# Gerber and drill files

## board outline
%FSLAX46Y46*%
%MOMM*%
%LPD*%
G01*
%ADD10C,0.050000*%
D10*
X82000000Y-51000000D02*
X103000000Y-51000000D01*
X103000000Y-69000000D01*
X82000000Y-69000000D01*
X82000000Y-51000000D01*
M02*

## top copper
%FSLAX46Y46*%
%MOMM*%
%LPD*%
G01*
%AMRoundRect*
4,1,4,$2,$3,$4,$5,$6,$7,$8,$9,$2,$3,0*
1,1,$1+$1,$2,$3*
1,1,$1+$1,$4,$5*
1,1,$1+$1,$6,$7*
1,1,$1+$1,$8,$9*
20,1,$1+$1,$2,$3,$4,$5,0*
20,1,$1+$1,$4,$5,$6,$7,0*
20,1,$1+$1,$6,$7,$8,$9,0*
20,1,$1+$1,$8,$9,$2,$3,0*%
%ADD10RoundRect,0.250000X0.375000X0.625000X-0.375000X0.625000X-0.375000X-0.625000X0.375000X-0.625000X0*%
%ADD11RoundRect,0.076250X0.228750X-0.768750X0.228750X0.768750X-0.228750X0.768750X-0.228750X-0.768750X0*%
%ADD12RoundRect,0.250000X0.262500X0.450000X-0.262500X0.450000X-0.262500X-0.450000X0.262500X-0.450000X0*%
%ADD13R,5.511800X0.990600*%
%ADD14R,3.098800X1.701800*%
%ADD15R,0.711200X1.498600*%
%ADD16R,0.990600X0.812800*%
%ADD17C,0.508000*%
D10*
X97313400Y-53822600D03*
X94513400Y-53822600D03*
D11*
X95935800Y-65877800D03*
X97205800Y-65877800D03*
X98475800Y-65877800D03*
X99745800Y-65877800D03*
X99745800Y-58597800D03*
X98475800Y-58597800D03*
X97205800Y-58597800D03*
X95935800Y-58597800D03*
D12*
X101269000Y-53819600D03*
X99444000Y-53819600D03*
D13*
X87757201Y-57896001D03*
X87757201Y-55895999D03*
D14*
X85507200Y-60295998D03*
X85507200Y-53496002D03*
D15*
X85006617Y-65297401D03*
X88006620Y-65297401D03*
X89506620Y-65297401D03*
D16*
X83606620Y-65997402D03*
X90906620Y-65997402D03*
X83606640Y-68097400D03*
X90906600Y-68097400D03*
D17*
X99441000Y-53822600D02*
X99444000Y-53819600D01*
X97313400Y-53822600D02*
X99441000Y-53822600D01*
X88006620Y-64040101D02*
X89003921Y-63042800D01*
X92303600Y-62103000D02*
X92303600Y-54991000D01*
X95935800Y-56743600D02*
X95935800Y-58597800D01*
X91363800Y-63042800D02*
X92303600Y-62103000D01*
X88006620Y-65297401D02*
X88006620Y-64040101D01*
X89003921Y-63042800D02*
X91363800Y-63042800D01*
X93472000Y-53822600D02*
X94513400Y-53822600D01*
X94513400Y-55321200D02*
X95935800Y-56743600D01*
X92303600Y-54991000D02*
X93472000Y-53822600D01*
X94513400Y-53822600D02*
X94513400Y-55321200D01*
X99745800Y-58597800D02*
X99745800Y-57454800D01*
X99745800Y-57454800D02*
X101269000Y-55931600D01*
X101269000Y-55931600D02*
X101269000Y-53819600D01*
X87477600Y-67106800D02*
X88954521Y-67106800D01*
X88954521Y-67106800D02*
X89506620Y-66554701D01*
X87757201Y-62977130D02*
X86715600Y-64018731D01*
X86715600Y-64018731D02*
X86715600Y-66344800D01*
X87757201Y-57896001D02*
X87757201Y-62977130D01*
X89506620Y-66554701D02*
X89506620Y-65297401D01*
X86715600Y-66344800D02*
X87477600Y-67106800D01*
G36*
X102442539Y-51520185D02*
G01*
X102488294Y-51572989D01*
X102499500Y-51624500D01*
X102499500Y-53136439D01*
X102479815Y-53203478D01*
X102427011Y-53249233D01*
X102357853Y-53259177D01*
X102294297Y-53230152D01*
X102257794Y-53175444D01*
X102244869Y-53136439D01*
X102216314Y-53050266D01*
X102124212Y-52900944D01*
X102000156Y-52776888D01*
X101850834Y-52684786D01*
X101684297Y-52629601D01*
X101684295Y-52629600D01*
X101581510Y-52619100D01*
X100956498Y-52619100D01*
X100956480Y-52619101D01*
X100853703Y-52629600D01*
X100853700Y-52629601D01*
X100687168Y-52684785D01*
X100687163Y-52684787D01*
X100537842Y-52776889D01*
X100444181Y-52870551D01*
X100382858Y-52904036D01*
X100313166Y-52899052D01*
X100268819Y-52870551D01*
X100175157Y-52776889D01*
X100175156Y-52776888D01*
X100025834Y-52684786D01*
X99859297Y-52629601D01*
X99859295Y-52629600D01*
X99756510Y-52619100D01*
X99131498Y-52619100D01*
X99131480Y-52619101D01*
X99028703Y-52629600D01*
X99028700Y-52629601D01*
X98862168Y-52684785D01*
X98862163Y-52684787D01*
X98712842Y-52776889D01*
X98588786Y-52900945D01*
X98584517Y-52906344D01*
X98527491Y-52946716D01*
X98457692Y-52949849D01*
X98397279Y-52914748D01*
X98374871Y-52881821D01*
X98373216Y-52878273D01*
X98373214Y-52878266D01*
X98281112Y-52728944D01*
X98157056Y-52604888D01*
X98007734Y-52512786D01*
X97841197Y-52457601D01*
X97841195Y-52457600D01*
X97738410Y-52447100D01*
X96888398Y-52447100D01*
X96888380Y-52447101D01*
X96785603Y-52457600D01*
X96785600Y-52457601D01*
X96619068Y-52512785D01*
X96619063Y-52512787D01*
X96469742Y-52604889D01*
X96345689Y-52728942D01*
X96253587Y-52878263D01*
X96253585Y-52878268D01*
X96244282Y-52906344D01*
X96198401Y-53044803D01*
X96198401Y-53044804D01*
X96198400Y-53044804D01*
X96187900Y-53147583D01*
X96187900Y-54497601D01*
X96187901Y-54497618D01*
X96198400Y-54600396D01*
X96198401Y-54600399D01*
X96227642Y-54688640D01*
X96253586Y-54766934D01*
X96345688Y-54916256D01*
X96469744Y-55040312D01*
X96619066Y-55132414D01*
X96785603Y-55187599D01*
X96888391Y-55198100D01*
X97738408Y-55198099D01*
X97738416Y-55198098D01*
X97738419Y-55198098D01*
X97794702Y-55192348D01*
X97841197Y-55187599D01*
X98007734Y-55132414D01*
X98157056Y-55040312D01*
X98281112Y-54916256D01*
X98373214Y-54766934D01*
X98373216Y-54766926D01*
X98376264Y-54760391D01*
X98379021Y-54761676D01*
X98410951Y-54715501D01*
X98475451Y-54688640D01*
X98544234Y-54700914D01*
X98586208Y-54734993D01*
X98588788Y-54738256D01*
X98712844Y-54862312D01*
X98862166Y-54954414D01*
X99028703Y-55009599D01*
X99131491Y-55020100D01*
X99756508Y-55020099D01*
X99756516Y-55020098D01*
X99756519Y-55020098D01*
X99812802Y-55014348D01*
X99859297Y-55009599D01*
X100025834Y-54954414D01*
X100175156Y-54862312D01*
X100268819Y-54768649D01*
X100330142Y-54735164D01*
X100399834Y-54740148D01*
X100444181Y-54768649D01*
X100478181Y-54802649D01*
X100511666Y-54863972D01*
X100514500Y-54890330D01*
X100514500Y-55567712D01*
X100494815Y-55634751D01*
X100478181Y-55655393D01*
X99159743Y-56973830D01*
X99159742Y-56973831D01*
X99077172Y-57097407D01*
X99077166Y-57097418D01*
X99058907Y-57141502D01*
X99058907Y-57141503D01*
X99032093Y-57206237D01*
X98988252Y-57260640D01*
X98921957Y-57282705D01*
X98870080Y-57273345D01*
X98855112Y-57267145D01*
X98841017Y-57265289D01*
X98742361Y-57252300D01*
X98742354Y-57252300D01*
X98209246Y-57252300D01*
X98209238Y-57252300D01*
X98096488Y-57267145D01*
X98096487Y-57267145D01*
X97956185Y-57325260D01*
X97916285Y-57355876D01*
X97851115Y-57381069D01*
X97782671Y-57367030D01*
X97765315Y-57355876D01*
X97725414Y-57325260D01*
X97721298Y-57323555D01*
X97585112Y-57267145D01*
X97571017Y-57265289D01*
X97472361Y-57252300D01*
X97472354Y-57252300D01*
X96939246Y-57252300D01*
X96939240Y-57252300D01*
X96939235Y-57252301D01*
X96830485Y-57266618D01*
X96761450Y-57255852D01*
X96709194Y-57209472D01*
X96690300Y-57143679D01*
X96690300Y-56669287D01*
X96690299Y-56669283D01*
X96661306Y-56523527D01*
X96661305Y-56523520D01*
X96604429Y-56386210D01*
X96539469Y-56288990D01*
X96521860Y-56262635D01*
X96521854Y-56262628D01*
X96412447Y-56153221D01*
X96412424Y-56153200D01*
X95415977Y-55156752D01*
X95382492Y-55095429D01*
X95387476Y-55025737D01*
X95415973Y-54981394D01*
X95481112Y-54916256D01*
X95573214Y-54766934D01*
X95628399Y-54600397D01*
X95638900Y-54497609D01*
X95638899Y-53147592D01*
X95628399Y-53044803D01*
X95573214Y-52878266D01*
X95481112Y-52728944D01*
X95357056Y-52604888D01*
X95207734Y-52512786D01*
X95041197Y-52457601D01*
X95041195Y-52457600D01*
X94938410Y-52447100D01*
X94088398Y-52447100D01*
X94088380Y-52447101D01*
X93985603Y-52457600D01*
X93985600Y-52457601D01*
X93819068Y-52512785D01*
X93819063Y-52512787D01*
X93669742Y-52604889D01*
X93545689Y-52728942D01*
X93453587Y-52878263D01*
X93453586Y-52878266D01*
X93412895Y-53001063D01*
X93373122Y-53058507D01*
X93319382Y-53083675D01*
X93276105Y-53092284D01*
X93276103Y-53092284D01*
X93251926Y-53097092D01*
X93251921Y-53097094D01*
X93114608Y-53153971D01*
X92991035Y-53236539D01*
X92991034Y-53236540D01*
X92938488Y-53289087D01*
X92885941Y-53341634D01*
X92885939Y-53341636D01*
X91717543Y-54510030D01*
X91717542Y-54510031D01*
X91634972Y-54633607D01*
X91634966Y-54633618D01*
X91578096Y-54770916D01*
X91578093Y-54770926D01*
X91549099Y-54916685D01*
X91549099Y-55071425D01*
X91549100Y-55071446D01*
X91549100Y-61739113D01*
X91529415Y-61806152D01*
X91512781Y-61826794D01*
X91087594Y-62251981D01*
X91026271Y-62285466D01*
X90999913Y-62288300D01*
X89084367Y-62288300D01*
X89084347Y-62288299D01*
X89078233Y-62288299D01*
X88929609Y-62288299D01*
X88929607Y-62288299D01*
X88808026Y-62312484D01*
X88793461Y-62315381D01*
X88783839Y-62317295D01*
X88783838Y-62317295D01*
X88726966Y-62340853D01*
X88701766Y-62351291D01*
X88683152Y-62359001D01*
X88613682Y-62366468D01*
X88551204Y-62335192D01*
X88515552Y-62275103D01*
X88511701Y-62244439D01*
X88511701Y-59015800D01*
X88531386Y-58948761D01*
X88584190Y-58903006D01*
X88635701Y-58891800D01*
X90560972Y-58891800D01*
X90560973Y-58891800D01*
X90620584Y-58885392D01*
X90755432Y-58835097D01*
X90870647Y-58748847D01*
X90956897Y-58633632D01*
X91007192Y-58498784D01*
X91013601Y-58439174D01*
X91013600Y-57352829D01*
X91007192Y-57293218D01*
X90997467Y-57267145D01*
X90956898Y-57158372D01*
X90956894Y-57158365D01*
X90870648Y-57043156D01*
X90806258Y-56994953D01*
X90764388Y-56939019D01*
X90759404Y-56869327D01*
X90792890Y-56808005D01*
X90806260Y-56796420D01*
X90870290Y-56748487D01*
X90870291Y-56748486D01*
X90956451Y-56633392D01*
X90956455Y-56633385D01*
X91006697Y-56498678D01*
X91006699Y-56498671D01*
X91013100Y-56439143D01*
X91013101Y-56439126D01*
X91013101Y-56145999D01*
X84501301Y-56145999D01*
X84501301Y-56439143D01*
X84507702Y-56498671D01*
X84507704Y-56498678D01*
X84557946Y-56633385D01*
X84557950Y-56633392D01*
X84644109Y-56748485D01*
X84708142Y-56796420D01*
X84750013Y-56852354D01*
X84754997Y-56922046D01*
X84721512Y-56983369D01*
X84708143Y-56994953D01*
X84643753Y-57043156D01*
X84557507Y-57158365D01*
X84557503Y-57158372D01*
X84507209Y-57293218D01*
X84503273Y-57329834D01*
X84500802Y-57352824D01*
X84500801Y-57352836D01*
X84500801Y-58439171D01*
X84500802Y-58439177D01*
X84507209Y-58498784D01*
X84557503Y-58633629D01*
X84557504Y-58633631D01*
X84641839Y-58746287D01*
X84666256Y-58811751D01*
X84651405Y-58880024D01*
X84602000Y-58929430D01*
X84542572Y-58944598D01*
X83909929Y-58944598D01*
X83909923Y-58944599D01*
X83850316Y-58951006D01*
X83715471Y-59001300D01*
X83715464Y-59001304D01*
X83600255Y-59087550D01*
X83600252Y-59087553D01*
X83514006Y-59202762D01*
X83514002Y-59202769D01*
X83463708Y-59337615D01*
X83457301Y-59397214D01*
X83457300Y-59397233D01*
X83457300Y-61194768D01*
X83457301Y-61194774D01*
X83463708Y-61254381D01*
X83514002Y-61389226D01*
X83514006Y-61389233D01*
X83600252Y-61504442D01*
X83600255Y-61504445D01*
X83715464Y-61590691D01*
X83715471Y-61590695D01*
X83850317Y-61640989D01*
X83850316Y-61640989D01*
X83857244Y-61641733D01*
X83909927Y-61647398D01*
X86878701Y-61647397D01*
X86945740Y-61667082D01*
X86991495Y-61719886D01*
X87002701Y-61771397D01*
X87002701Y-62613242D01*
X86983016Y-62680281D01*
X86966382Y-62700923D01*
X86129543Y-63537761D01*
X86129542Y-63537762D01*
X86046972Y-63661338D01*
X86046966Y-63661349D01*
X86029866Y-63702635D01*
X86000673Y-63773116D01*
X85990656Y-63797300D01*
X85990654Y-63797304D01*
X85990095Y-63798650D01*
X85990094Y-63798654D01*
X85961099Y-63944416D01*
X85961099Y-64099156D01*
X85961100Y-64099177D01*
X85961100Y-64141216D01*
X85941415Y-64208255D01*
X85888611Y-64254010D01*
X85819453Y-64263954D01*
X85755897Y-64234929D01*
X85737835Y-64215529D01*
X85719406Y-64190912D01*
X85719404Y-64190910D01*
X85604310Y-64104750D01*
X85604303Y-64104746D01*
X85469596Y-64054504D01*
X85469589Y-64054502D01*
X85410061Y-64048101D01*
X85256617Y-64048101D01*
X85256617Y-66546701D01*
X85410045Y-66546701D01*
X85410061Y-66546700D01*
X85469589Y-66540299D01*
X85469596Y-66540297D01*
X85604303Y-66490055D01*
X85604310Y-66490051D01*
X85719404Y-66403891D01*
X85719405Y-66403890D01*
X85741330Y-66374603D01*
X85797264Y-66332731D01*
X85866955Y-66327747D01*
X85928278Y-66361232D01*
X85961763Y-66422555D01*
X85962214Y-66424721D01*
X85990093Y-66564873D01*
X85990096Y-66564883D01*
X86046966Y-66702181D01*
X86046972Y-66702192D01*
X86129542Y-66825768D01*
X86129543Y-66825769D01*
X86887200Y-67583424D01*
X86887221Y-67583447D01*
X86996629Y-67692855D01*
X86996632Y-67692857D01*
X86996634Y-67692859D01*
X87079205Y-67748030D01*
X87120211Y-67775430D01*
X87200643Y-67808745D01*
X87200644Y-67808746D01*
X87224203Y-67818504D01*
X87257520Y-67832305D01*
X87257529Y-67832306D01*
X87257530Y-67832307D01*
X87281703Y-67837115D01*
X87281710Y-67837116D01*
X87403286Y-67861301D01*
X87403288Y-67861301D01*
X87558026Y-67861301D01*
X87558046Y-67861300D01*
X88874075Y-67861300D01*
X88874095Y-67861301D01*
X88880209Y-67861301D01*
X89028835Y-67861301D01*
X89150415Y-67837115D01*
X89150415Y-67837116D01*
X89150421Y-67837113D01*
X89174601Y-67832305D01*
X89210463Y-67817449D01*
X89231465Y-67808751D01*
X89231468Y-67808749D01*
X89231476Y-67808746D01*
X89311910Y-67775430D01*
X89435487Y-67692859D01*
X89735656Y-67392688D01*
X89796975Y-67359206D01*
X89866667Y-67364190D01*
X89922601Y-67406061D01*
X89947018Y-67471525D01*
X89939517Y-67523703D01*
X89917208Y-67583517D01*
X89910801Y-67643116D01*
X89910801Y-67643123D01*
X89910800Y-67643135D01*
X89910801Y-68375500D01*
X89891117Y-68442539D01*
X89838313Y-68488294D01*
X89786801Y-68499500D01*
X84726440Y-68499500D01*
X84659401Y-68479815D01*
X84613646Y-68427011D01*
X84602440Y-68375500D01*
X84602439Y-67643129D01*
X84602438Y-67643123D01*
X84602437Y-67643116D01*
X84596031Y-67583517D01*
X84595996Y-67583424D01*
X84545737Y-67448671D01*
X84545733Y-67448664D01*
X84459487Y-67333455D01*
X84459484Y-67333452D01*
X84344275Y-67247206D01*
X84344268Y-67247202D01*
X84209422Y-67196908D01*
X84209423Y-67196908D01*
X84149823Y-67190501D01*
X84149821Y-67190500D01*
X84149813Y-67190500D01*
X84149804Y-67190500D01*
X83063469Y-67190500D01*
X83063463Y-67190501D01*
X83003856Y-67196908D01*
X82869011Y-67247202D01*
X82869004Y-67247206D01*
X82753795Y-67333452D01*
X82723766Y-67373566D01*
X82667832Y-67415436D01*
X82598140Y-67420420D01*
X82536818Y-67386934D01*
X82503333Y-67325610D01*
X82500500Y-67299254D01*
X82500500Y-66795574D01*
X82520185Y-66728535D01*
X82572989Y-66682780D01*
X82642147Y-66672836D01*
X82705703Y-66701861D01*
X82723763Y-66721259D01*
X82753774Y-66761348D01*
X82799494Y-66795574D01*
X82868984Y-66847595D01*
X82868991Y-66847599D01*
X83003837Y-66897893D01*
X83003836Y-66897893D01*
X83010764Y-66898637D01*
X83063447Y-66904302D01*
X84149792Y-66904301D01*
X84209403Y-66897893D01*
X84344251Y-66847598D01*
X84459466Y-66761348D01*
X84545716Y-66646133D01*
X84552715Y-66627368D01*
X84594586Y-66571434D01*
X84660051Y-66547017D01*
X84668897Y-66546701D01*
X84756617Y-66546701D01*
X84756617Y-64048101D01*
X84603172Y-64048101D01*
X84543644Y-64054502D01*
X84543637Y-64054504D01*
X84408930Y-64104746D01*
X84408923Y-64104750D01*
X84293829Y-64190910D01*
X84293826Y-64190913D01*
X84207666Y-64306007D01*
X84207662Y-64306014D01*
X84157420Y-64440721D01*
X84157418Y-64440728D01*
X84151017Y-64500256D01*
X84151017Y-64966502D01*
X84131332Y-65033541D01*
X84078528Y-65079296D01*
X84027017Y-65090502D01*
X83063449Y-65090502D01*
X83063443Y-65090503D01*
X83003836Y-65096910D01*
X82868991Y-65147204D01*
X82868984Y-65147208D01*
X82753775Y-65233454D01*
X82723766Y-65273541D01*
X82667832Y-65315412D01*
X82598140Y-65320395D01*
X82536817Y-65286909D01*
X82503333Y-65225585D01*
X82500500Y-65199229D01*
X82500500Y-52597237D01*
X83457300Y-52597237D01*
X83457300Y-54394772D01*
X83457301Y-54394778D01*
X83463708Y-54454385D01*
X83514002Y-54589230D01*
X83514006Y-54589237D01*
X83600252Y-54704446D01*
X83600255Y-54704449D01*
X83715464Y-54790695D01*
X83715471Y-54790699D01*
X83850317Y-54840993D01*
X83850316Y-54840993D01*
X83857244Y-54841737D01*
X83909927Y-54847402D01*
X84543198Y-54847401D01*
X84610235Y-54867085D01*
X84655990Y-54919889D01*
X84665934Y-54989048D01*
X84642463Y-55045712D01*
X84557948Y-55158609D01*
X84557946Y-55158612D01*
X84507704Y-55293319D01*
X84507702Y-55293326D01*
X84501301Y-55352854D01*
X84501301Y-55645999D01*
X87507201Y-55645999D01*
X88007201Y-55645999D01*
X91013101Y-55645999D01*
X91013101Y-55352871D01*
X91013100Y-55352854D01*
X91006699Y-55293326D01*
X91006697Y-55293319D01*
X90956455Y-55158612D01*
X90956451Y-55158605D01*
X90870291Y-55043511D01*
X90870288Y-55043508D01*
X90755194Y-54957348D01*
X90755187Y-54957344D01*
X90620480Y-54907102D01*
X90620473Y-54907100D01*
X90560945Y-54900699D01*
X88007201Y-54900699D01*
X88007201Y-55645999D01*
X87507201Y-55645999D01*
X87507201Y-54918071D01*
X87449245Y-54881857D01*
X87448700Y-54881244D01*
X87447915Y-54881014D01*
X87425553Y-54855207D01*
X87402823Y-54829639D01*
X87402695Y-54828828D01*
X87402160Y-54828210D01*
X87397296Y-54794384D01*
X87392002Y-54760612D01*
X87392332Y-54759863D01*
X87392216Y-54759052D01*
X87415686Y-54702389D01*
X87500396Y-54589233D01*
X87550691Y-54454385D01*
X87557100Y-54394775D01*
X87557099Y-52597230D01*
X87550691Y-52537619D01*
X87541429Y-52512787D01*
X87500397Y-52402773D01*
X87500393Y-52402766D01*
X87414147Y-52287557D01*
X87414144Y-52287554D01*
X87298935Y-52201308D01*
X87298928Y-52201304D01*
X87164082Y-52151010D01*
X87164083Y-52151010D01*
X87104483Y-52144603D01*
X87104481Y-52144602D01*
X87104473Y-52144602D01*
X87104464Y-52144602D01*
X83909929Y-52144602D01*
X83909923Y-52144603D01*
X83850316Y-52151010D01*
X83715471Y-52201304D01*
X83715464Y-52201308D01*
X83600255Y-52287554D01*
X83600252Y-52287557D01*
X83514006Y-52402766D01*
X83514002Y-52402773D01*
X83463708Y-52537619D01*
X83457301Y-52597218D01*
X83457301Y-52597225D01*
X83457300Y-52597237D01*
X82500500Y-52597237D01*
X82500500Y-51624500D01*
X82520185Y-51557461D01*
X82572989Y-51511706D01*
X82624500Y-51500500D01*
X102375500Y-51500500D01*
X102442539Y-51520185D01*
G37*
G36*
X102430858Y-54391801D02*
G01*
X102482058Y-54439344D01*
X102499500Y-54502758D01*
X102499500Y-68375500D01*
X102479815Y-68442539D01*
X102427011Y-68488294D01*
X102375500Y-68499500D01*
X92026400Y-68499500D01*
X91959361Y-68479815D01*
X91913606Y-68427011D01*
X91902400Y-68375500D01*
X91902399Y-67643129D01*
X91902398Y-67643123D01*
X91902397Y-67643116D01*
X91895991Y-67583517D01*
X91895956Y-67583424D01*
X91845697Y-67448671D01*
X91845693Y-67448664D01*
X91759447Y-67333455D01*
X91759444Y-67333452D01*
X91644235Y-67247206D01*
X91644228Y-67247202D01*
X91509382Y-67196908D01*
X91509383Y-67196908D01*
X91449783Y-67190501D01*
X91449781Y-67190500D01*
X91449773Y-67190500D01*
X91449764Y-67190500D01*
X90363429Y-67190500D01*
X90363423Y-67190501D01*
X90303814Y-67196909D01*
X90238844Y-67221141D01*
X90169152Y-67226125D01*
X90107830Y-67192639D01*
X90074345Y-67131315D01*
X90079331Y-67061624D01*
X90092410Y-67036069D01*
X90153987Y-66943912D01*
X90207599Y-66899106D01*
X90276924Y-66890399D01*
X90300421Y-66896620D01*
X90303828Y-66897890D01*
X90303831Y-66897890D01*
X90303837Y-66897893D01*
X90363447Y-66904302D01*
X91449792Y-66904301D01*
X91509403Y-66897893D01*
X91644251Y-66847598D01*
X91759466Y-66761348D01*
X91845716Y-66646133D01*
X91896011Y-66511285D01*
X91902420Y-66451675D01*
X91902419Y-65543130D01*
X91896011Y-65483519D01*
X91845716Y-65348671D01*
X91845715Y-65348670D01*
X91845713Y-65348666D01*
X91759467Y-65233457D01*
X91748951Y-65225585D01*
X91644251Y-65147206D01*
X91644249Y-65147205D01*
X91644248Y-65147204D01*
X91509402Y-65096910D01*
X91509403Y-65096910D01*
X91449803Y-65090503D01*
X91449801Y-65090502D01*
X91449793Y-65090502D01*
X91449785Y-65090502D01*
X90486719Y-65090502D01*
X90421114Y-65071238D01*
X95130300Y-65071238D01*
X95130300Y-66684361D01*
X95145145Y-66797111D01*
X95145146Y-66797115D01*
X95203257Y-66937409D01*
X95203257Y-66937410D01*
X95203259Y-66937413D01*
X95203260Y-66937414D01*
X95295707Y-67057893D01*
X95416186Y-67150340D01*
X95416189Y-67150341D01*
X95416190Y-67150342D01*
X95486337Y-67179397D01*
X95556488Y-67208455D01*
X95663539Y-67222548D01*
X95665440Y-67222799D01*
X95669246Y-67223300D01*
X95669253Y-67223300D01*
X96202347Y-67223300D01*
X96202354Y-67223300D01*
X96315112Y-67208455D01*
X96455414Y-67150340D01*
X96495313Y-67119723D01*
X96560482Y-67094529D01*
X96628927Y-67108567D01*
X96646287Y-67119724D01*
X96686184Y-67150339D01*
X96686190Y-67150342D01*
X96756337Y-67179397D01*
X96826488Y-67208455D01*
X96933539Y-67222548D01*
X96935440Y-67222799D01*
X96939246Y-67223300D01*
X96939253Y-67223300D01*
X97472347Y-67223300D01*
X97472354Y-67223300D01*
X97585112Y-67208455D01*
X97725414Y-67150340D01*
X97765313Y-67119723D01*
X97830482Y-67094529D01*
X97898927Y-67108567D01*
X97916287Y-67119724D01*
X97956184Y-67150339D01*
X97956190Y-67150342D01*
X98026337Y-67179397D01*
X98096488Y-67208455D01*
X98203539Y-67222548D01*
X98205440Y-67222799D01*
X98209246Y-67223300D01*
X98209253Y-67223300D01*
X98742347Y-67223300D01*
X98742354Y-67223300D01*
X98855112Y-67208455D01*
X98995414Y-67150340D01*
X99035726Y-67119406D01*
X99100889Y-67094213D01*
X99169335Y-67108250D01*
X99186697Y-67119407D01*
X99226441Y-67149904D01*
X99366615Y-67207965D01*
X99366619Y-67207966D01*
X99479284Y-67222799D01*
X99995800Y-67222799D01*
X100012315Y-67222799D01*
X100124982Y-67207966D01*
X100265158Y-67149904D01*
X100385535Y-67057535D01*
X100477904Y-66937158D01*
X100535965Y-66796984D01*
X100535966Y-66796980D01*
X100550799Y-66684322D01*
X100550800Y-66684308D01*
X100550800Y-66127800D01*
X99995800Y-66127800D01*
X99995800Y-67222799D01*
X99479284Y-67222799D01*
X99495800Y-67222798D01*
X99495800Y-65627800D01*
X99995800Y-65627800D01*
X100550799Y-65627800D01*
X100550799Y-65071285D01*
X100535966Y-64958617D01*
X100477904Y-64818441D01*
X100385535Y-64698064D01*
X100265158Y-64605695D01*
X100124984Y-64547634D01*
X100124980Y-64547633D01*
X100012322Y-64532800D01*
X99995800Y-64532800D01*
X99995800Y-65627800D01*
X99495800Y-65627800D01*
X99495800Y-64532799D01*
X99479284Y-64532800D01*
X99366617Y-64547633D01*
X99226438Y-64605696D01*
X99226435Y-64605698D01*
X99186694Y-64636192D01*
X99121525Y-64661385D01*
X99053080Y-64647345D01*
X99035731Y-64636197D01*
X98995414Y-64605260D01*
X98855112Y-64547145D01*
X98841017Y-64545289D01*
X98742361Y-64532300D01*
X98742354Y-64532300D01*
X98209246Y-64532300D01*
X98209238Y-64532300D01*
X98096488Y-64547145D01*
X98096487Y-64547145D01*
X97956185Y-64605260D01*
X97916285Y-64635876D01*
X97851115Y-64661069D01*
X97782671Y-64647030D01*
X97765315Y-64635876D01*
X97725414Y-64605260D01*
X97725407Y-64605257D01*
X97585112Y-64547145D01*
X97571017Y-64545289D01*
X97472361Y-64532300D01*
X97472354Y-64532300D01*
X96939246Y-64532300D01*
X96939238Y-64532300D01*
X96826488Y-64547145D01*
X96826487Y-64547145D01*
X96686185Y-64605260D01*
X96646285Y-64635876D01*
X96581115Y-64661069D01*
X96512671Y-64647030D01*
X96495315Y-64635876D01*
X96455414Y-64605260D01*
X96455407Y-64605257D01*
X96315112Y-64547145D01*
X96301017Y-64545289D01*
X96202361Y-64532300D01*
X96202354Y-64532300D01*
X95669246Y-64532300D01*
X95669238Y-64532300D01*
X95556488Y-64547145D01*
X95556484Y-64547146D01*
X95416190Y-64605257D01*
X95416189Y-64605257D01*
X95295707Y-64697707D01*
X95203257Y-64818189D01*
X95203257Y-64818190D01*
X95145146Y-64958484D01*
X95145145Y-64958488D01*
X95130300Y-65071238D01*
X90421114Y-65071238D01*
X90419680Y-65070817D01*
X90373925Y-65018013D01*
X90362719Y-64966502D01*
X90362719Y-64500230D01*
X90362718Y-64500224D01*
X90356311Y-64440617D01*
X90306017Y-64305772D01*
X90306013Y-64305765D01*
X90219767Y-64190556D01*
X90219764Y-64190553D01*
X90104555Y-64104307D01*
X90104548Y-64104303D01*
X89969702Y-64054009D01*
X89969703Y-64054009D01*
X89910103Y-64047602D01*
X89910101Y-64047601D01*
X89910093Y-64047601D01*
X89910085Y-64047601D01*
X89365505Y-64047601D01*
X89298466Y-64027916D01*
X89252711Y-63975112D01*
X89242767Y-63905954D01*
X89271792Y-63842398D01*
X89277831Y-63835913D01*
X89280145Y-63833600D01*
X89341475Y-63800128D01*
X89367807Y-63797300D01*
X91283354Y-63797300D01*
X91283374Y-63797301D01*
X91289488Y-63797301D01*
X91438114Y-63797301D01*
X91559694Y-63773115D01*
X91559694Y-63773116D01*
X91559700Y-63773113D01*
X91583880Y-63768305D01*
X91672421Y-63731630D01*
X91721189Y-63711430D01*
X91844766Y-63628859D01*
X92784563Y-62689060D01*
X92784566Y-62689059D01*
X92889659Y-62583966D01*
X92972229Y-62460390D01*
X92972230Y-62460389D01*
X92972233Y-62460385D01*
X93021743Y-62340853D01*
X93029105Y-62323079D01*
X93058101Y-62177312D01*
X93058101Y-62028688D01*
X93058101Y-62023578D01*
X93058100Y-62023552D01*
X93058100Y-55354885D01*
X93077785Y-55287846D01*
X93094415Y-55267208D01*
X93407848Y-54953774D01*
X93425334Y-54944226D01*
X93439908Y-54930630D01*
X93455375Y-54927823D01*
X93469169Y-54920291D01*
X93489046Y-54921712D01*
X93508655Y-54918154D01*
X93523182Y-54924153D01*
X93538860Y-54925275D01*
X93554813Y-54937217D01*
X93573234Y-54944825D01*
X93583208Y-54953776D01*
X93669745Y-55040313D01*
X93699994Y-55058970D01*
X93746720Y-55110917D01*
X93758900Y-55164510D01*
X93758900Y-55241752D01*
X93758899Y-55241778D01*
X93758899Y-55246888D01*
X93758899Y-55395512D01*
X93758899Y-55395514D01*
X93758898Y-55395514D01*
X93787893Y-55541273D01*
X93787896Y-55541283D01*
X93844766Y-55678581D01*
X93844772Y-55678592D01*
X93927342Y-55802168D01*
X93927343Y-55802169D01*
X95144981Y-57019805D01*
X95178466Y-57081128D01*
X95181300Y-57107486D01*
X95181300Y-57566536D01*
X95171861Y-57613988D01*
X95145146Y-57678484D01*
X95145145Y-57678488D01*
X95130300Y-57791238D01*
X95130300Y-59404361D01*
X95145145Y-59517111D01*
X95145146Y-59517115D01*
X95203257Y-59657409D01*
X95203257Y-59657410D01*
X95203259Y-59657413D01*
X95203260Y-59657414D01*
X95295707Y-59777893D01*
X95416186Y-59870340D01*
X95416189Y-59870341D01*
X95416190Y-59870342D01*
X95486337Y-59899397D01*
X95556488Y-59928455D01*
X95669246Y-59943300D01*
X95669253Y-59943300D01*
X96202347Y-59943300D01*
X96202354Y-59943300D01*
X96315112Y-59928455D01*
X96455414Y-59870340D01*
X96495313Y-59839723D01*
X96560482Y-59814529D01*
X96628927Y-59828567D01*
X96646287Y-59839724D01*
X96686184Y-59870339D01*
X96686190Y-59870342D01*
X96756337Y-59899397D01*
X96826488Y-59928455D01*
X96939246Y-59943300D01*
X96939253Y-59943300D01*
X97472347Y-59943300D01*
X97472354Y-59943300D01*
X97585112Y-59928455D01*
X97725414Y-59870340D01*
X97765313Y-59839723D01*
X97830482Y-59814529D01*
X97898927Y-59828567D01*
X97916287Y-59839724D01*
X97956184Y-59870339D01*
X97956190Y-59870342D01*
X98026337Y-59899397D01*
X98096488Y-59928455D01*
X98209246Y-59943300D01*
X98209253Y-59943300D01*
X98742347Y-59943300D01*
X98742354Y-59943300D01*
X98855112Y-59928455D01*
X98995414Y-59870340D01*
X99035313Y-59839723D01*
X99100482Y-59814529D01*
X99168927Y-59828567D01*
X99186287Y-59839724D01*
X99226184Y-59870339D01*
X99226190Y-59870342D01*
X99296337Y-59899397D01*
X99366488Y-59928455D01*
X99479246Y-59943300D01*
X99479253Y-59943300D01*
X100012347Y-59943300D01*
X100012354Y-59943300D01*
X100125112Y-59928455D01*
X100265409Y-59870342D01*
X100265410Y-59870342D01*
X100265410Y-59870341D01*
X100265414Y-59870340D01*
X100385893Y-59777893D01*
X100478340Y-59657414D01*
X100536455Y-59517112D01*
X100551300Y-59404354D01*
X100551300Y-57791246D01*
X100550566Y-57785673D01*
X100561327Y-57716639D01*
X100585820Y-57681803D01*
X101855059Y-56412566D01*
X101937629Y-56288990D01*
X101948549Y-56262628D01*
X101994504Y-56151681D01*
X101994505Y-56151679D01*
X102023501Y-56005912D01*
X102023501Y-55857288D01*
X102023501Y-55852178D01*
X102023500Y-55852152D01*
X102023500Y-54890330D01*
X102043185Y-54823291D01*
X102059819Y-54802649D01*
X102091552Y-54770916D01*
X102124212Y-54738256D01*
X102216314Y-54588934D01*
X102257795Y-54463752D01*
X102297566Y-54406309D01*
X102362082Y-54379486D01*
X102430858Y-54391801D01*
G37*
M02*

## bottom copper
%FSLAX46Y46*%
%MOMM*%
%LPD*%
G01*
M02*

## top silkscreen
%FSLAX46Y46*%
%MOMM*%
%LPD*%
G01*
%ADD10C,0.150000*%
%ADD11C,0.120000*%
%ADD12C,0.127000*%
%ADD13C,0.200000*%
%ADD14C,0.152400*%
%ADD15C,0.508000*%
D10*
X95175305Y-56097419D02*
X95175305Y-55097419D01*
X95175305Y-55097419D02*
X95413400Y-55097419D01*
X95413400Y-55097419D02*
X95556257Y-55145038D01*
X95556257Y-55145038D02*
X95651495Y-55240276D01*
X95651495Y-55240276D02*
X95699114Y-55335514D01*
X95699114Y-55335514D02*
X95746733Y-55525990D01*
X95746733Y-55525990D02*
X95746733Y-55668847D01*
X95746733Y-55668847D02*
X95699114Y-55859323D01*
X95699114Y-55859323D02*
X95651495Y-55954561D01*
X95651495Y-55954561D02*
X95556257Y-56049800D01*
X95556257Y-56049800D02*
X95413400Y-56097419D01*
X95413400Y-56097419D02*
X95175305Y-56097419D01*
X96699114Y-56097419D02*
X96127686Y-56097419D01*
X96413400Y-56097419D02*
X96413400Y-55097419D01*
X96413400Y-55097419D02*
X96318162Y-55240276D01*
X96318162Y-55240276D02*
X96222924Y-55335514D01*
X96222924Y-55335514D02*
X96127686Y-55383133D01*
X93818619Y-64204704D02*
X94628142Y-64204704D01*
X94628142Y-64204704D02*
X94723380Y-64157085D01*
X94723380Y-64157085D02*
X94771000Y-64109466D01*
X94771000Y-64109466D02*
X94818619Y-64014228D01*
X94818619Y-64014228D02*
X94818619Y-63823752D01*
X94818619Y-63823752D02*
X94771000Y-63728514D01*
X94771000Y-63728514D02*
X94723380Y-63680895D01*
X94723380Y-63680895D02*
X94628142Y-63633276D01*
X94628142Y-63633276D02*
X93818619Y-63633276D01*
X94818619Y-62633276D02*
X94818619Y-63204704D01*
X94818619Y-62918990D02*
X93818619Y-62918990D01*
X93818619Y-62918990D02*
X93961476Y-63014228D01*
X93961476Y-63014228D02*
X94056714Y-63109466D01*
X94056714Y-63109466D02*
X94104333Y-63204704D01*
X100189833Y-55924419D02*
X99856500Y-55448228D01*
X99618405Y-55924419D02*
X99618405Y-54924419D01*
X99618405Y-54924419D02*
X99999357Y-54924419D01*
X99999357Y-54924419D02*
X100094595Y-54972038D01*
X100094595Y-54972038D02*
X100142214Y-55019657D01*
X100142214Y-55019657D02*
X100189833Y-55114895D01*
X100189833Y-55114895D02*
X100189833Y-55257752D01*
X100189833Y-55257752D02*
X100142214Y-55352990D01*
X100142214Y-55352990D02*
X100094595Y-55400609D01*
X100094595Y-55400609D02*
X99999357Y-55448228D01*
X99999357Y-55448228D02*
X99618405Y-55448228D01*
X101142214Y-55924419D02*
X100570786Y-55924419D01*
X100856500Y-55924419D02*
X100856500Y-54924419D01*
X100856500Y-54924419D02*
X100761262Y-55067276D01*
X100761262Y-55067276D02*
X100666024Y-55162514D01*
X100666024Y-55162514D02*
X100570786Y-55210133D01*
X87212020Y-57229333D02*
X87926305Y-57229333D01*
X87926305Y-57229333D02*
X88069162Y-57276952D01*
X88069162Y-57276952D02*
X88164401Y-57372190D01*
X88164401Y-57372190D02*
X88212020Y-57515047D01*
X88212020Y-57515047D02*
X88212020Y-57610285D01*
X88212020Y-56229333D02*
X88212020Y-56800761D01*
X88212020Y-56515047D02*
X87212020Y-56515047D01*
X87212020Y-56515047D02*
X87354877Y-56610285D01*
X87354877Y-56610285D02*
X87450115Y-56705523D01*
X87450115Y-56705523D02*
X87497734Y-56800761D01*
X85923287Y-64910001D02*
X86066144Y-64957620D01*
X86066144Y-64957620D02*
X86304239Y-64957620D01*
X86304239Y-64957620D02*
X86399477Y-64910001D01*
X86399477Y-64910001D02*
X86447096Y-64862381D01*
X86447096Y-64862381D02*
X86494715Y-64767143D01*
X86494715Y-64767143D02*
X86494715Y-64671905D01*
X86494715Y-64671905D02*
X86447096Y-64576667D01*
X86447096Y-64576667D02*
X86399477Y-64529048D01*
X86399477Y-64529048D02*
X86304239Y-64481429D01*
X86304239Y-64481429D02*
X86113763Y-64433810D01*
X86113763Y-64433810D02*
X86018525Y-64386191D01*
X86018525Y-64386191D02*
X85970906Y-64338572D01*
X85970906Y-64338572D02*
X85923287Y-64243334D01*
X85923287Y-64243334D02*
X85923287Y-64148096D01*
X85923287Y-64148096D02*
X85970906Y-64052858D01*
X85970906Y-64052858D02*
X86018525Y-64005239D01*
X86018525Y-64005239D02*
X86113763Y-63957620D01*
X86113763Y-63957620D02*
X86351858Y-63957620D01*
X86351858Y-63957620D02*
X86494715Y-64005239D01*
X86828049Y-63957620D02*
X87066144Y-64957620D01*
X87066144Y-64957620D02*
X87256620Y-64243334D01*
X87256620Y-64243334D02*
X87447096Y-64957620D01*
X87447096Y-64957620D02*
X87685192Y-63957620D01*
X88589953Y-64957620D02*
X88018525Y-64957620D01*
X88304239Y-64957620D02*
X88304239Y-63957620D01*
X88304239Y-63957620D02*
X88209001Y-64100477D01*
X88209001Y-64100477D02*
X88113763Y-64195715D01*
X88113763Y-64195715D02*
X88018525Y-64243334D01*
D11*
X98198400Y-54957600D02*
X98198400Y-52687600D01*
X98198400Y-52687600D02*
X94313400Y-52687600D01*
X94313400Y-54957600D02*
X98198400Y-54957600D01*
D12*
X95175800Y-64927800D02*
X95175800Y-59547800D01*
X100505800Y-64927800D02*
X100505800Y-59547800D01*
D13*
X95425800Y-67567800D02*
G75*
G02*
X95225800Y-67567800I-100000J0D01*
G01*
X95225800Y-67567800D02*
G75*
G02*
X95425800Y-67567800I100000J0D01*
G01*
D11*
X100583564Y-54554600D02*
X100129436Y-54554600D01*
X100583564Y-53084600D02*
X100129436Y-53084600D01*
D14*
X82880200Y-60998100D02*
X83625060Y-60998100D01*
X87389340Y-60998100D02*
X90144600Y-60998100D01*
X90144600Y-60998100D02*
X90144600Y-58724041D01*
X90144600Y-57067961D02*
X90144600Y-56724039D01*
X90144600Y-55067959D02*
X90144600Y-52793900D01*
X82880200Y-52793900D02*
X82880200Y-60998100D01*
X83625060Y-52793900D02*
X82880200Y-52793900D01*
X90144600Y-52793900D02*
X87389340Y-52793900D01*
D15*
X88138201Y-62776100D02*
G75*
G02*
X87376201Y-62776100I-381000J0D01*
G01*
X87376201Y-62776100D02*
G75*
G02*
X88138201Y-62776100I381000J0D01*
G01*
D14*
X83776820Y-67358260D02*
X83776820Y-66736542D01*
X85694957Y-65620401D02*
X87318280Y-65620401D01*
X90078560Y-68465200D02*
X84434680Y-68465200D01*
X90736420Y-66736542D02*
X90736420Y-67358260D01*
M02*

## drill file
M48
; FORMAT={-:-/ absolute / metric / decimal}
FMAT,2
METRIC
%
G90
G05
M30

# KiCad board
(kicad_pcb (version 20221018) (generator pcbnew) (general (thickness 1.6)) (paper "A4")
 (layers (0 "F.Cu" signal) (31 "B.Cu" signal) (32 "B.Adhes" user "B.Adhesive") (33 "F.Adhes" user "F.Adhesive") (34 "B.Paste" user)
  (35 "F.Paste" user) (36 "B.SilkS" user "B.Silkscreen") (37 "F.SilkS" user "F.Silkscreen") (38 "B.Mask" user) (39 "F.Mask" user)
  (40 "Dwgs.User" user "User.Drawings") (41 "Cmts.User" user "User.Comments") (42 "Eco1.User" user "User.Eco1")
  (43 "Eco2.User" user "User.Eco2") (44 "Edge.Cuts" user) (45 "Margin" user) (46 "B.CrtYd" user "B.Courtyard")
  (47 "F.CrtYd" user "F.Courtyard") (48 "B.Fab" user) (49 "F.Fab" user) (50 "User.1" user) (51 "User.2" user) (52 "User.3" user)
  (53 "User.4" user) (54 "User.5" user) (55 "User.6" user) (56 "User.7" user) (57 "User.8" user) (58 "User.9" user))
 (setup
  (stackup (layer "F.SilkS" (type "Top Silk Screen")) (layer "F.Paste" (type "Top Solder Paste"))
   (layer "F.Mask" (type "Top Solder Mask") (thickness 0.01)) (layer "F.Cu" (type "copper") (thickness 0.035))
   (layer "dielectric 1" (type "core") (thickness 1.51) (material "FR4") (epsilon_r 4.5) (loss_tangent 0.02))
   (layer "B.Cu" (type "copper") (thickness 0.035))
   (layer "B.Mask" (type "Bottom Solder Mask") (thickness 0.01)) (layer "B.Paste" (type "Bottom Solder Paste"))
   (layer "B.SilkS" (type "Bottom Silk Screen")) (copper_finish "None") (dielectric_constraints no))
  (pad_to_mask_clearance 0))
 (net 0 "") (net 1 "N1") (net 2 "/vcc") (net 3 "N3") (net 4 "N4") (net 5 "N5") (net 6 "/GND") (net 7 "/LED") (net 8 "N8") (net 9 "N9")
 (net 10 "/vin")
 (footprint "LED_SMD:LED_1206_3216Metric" (layer "F.Cu") (at 95.9134 53.8226 180)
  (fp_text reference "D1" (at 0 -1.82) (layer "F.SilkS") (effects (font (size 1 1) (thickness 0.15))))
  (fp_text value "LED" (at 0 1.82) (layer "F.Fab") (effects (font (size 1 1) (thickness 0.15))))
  (fp_line (start -2.285 -1.135) (end -2.285 1.135) (stroke (width 0.12) (type solid)) (layer "F.SilkS"))
  (fp_line (start -2.285 1.135) (end 1.6 1.135) (stroke (width 0.12) (type solid)) (layer "F.SilkS"))
  (fp_line (start 1.6 -1.135) (end -2.285 -1.135) (stroke (width 0.12) (type solid)) (layer "F.SilkS"))
  (pad "1" smd roundrect (at -1.4 0 180) (size 1.25 1.75) (layers "F.Cu" "F.Paste" "F.Mask") (roundrect_rratio 0.2) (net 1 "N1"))
  (pad "2" smd roundrect (at 1.4 0 180) (size 1.25 1.75) (layers "F.Cu" "F.Paste" "F.Mask") (roundrect_rratio 0.2) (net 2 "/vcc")))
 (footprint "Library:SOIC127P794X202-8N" (layer "F.Cu") (at 97.8408 62.2378 90)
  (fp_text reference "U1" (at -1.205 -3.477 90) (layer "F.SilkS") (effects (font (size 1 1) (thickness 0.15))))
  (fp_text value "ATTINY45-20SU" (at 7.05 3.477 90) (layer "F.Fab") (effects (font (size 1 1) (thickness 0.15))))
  (fp_line (start -2.69 -2.665) (end 2.69 -2.665) (stroke (width 0.127) (type solid)) (layer "F.SilkS"))
  (fp_line (start -2.69 2.665) (end 2.69 2.665) (stroke (width 0.127) (type solid)) (layer "F.SilkS"))
  (fp_circle (center -5.33 -2.515) (end -5.23 -2.515) (stroke (width 0.2) (type solid)) (fill none) (layer "F.SilkS"))
  (pad "1" smd roundrect (at -3.64 -1.905 90) (size 1.69 0.61) (layers "F.Cu" "F.Paste" "F.Mask") (roundrect_rratio 0.125) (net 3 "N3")
   (solder_mask_margin 0.102))
  (pad "2" smd roundrect (at -3.64 -0.635 90) (size 1.69 0.61) (layers "F.Cu" "F.Paste" "F.Mask") (roundrect_rratio 0.125) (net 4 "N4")
   (solder_mask_margin 0.102))
  (pad "3" smd roundrect (at -3.64 0.635 90) (size 1.69 0.61) (layers "F.Cu" "F.Paste" "F.Mask") (roundrect_rratio 0.125) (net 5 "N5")
   (solder_mask_margin 0.102))
  (pad "4" smd roundrect (at -3.64 1.905 90) (size 1.69 0.61) (layers "F.Cu" "F.Paste" "F.Mask") (roundrect_rratio 0.125) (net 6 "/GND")
   (solder_mask_margin 0.102))
  (pad "5" smd roundrect (at 3.64 1.905 90) (size 1.69 0.61) (layers "F.Cu" "F.Paste" "F.Mask") (roundrect_rratio 0.125) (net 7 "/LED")
   (solder_mask_margin 0.102))
  (pad "6" smd roundrect (at 3.64 0.635 90) (size 1.69 0.61) (layers "F.Cu" "F.Paste" "F.Mask") (roundrect_rratio 0.125) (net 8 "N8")
   (solder_mask_margin 0.102))
  (pad "7" smd roundrect (at 3.64 -0.635 90) (size 1.69 0.61) (layers "F.Cu" "F.Paste" "F.Mask") (roundrect_rratio 0.125) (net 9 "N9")
   (solder_mask_margin 0.102))
  (pad "8" smd roundrect (at 3.64 -1.905 90) (size 1.69 0.61) (layers "F.Cu" "F.Paste" "F.Mask") (roundrect_rratio 0.125) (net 2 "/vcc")
   (solder_mask_margin 0.102)))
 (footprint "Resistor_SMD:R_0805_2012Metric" (layer "F.Cu") (at 100.3565 53.8196 180)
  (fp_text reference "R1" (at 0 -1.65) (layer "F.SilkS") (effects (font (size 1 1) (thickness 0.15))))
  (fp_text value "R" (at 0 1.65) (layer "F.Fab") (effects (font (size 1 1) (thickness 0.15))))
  (fp_line (start -0.227064 -0.735) (end 0.227064 -0.735) (stroke (width 0.12) (type solid)) (layer "F.SilkS"))
  (fp_line (start -0.227064 0.735) (end 0.227064 0.735) (stroke (width 0.12) (type solid)) (layer "F.SilkS"))
  (pad "1" smd roundrect (at -0.9125 0 180) (size 1.025 1.4) (layers "F.Cu" "F.Paste" "F.Mask") (roundrect_rratio 0.243902) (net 7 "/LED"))
  (pad "2" smd roundrect (at 0.9125 0 180) (size 1.025 1.4) (layers "F.Cu" "F.Paste" "F.Mask") (roundrect_rratio 0.243902) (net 1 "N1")))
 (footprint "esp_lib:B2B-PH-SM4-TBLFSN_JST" (layer "F.Cu") (at 86.5124 56.896 90)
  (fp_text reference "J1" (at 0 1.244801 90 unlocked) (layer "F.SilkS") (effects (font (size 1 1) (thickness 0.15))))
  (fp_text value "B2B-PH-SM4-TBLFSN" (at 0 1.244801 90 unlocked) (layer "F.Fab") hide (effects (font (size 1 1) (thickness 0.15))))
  (fp_line (start -4.1021 -3.6322) (end -4.1021 -2.88734) (stroke (width 0.1524) (type solid)) (layer "F.SilkS"))
  (fp_line (start -4.1021 0.87694) (end -4.1021 3.6322) (stroke (width 0.1524) (type solid)) (layer "F.SilkS"))
  (fp_line (start -4.1021 3.6322) (end -1.828041 3.6322) (stroke (width 0.1524) (type solid)) (layer "F.SilkS"))
  (fp_line (start -0.171961 3.6322) (end 0.171961 3.6322) (stroke (width 0.1524) (type solid)) (layer "F.SilkS"))
  (fp_line (start 1.828041 3.6322) (end 4.1021 3.6322) (stroke (width 0.1524) (type solid)) (layer "F.SilkS"))
  (fp_line (start 4.1021 -3.6322) (end -4.1021 -3.6322) (stroke (width 0.1524) (type solid)) (layer "F.SilkS"))
  (fp_line (start 4.1021 -2.88734) (end 4.1021 -3.6322) (stroke (width 0.1524) (type solid)) (layer "F.SilkS"))
  (fp_line (start 4.1021 3.6322) (end 4.1021 0.87694) (stroke (width 0.1524) (type solid)) (layer "F.SilkS"))
  (fp_circle (center -5.8801 1.244801) (end -5.4991 1.244801) (stroke (width 0.508) (type solid)) (fill none) (layer "F.SilkS"))
  (pad "1" smd rect (at -1.000001 1.244801 90) (size 0.9906 5.5118) (layers "F.Cu" "F.Paste" "F.Mask") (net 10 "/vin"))
  (pad "2" smd rect (at 1.000001 1.244801 90) (size 0.9906 5.5118) (layers "F.Cu" "F.Paste" "F.Mask") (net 6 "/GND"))
  (pad "3" smd rect (at -3.399998 -1.0052 180) (size 3.0988 1.7018) (layers "F.Cu" "F.Paste" "F.Mask"))
  (pad "4" smd rect (at 3.399998 -1.0052 180) (size 3.0988 1.7018) (layers "F.Cu" "F.Paste" "F.Mask")))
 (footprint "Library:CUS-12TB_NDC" (layer "F.Cu") (at 87.25662 67.042801)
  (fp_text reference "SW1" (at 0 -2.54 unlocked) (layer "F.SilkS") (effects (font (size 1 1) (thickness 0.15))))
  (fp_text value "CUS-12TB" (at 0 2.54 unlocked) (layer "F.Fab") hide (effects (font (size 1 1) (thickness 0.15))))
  (fp_line (start -3.4798 0.315459) (end -3.4798 -0.306259) (stroke (width 0.1524) (type solid)) (layer "F.SilkS"))
  (fp_line (start -1.561663 -1.4224) (end 0.06166 -1.4224) (stroke (width 0.1524) (type solid)) (layer "F.SilkS"))
  (fp_line (start 2.82194 1.422399) (end -2.82194 1.422399) (stroke (width 0.1524) (type solid)) (layer "F.SilkS"))
  (fp_line (start 3.4798 -0.306259) (end 3.4798 0.315459) (stroke (width 0.1524) (type solid)) (layer "F.SilkS"))
  (pad "1" smd rect (at -2.250003 -1.7454) (size 0.7112 1.4986) (layers "F.Cu" "F.Paste" "F.Mask") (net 6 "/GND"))
  (pad "2" smd rect (at 0.75 -1.7454) (size 0.7112 1.4986) (layers "F.Cu" "F.Paste" "F.Mask") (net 2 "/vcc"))
  (pad "3" smd rect (at 2.25 -1.7454) (size 0.7112 1.4986) (layers "F.Cu" "F.Paste" "F.Mask") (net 10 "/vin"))
  (pad "4" smd rect (at -3.65 -1.045399) (size 0.9906 0.8128) (layers "F.Cu" "F.Paste" "F.Mask"))
  (pad "5" smd rect (at 3.65 -1.045399) (size 0.9906 0.8128) (layers "F.Cu" "F.Paste" "F.Mask"))
  (pad "6" smd rect (at -3.64998 1.054599) (size 0.9906 0.8128) (layers "F.Cu" "F.Paste" "F.Mask"))
  (pad "7" smd rect (at 3.64998 1.054599) (size 0.9906 0.8128) (layers "F.Cu" "F.Paste" "F.Mask")))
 (gr_rect (start 82 51) (end 103 69) (stroke (width 0.05) (type default)) (fill none) (layer "Edge.Cuts"))
 (segment (start 99.441 53.8226) (end 99.444 53.8196) (width 0.508) (layer "F.Cu") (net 1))
 (segment (start 97.3134 53.8226) (end 99.441 53.8226) (width 0.508) (layer "F.Cu") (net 1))
 (segment (start 88.00662 64.040101) (end 89.003921 63.0428) (width 0.508) (layer "F.Cu") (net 2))
 (segment (start 92.3036 62.103) (end 92.3036 54.991) (width 0.508) (layer "F.Cu") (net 2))
 (segment (start 95.9358 56.7436) (end 95.9358 58.5978) (width 0.508) (layer "F.Cu") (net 2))
 (segment (start 91.3638 63.0428) (end 92.3036 62.103) (width 0.508) (layer "F.Cu") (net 2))
 (segment (start 88.00662 65.297401) (end 88.00662 64.040101) (width 0.508) (layer "F.Cu") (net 2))
 (segment (start 89.003921 63.0428) (end 91.3638 63.0428) (width 0.508) (layer "F.Cu") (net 2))
 (segment (start 93.472 53.8226) (end 94.5134 53.8226) (width 0.508) (layer "F.Cu") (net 2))
 (segment (start 94.5134 55.3212) (end 95.9358 56.7436) (width 0.508) (layer "F.Cu") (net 2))
 (segment (start 92.3036 54.991) (end 93.472 53.8226) (width 0.508) (layer "F.Cu") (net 2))
 (segment (start 94.5134 53.8226) (end 94.5134 55.3212) (width 0.508) (layer "F.Cu") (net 2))
 (segment (start 99.7458 58.5978) (end 99.7458 57.4548) (width 0.508) (layer "F.Cu") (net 7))
 (segment (start 99.7458 57.4548) (end 101.269 55.9316) (width 0.508) (layer "F.Cu") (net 7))
 (segment (start 101.269 55.9316) (end 101.269 53.8196) (width 0.508) (layer "F.Cu") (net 7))
 (segment (start 87.4776 67.1068) (end 88.954521 67.1068) (width 0.508) (layer "F.Cu") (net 10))
 (segment (start 88.954521 67.1068) (end 89.50662 66.554701) (width 0.508) (layer "F.Cu") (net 10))
 (segment (start 87.757201 62.97713) (end 86.7156 64.018731) (width 0.508) (layer "F.Cu") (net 10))
 (segment (start 86.7156 64.018731) (end 86.7156 66.3448) (width 0.508) (layer "F.Cu") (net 10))
 (segment (start 87.757201 57.896001) (end 87.757201 62.97713) (width 0.508) (layer "F.Cu") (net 10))
 (segment (start 89.50662 66.554701) (end 89.50662 65.297401) (width 0.508) (layer "F.Cu") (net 10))
 (segment (start 86.7156 66.3448) (end 87.4776 67.1068) (width 0.508) (layer "F.Cu") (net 10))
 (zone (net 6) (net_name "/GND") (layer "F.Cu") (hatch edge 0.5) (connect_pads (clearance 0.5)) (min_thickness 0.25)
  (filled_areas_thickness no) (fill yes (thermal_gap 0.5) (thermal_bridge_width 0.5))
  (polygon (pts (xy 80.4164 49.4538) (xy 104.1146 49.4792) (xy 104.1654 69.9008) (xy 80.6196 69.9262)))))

